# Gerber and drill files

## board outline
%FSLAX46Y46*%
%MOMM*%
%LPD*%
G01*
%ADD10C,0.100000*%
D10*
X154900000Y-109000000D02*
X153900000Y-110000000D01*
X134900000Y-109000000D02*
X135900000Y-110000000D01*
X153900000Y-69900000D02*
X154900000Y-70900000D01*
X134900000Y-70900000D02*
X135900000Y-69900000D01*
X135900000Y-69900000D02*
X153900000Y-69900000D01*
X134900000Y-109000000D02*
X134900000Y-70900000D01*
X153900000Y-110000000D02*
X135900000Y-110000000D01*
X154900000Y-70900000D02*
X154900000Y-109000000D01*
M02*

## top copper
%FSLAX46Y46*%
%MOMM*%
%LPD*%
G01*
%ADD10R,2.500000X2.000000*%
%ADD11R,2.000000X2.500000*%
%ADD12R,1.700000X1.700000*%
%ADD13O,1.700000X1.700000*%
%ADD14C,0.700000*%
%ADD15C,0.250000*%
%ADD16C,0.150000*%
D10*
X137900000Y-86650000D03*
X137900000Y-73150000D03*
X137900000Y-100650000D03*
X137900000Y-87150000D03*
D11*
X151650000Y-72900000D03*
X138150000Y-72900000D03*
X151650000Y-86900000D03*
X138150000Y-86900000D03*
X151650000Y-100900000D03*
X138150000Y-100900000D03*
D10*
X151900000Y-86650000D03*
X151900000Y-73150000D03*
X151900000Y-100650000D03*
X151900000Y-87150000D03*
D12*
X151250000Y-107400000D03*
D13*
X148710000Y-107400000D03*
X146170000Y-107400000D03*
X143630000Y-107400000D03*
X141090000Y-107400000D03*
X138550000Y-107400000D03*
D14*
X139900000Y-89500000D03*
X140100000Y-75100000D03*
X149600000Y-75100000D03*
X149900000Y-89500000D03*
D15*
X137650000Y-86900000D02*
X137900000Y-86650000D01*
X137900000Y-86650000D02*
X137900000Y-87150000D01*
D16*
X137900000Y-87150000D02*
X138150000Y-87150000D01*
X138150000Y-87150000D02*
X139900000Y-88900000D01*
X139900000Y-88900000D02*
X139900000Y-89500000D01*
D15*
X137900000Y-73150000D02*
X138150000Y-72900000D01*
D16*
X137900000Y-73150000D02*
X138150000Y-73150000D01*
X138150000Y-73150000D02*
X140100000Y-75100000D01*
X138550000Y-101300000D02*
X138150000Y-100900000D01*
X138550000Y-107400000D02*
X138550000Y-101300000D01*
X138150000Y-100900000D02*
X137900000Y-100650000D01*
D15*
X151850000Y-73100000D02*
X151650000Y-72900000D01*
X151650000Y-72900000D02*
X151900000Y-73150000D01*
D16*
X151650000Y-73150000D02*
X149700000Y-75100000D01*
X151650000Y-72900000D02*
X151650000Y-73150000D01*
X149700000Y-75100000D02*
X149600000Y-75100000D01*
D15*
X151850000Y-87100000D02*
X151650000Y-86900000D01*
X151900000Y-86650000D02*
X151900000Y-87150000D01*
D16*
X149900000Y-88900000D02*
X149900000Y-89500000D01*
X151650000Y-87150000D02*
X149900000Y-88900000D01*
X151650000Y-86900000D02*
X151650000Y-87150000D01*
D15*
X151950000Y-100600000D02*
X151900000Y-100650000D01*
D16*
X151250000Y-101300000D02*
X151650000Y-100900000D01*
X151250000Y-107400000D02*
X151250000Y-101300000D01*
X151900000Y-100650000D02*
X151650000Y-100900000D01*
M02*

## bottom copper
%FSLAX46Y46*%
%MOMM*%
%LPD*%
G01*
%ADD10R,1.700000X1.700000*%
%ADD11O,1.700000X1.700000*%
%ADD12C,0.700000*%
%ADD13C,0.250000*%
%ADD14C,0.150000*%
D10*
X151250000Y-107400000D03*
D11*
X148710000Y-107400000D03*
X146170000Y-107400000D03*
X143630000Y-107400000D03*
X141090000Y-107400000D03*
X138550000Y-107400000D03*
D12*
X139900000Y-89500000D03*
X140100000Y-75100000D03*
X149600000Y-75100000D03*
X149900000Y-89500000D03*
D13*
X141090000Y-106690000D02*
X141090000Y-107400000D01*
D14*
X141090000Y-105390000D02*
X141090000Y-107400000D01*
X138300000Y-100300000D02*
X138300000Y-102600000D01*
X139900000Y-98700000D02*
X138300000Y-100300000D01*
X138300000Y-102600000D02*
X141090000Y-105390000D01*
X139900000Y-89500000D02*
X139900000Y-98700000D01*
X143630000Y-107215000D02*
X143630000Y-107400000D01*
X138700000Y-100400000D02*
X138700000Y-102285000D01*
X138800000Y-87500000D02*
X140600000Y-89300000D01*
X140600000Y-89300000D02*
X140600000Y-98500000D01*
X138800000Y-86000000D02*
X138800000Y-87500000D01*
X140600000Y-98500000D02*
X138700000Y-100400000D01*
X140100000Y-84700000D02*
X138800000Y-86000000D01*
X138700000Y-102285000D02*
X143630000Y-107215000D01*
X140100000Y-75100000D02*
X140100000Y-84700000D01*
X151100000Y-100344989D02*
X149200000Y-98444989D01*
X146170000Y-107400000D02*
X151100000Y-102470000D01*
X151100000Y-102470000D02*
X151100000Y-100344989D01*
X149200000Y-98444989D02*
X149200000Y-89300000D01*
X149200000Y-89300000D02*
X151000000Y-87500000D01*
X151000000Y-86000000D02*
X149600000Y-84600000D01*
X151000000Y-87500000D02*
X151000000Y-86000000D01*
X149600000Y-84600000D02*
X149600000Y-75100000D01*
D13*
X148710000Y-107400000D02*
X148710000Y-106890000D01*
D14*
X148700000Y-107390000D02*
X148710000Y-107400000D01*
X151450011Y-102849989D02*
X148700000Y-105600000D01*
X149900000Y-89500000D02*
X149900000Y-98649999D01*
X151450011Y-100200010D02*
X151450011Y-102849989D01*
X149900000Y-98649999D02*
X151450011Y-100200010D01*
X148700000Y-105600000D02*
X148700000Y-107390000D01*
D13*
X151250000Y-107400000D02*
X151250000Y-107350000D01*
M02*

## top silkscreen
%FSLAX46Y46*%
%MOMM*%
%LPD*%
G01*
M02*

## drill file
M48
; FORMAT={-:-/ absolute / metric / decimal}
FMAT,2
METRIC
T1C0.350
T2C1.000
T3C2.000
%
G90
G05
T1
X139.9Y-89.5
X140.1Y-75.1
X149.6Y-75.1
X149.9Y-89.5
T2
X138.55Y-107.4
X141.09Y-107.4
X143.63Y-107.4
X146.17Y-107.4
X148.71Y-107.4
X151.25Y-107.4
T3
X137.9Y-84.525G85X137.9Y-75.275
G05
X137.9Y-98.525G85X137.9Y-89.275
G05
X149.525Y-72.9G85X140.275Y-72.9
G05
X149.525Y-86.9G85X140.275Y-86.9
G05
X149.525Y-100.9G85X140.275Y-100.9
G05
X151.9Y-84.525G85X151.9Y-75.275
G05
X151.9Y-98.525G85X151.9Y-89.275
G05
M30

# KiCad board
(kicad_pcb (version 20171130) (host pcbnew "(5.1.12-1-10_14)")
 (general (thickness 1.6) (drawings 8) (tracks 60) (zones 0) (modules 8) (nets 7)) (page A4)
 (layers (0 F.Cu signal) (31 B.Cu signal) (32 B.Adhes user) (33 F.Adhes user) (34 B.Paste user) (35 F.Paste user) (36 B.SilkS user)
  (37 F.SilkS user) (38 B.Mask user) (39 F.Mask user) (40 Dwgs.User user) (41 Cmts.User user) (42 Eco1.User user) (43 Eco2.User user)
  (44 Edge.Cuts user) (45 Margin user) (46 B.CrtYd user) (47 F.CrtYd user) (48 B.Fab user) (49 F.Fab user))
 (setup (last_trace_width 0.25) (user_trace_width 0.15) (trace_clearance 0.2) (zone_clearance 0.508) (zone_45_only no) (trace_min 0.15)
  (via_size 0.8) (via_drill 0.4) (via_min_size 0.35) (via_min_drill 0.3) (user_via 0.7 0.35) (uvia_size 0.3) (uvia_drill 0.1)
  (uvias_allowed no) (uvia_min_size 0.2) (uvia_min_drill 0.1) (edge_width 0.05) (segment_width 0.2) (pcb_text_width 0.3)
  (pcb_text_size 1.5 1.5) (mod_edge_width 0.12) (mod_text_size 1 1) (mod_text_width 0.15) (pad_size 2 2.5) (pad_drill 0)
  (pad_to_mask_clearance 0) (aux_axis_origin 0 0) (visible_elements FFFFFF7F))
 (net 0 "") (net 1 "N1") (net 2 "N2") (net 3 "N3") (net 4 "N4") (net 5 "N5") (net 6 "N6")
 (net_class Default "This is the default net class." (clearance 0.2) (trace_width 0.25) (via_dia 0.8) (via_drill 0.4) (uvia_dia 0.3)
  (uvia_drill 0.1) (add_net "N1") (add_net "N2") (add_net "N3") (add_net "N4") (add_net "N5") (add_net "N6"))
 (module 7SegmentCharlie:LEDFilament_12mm (layer F.Cu) (at 137.9 79.9 90)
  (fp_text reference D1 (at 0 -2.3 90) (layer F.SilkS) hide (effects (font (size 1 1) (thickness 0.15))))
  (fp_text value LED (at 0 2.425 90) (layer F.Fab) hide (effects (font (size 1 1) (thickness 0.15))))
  (pad "" smd rect (at 6.75 0 90) (size 2 2.5) (layers F.Paste F.Mask))
  (pad "" smd rect (at -6.75 0 90) (size 2 2.5) (layers F.Paste F.Mask))
  (pad "" np_thru_hole oval (at 0 0 90) (size 11.25 2) (drill oval 11.25 2) (layers *.Cu *.Mask))
  (pad 1 smd rect (at -6.75 0 90) (size 2 2.5) (layers F.Cu) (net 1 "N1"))
  (pad 2 smd rect (at 6.75 0 90) (size 2 2.5) (layers F.Cu) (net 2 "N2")))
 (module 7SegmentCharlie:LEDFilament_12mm (layer F.Cu) (at 137.9 93.9 90)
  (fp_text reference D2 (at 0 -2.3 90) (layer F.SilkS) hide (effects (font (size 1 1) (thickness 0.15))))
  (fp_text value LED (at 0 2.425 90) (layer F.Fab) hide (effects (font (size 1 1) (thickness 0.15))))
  (pad "" smd rect (at 6.75 0 90) (size 2 2.5) (layers F.Paste F.Mask))
  (pad "" smd rect (at -6.75 0 90) (size 2 2.5) (layers F.Paste F.Mask))
  (pad "" np_thru_hole oval (at 0 0 90) (size 11.25 2) (drill oval 11.25 2) (layers *.Cu *.Mask))
  (pad 1 smd rect (at -6.75 0 90) (size 2 2.5) (layers F.Cu) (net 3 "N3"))
  (pad 2 smd rect (at 6.75 0 90) (size 2 2.5) (layers F.Cu) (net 1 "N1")))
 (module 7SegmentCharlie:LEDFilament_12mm (layer F.Cu) (at 144.9 72.9 180)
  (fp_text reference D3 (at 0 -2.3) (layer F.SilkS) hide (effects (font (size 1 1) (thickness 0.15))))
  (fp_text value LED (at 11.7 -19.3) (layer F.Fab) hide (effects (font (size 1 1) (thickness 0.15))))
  (pad "" smd rect (at 6.75 0 180) (size 2 2.5) (layers F.Paste F.Mask))
  (pad "" smd rect (at -6.75 0 180) (size 2 2.5) (layers F.Paste F.Mask))
  (pad "" np_thru_hole oval (at 0 0 180) (size 11.25 2) (drill oval 11.25 2) (layers *.Cu *.Mask))
  (pad 1 smd rect (at -6.75 0 180) (size 2 2.5) (layers F.Cu) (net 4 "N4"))
  (pad 2 smd rect (at 6.75 0 180) (size 2 2.5) (layers F.Cu) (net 2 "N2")))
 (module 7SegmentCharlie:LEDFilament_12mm (layer F.Cu) (at 144.9 86.9 180)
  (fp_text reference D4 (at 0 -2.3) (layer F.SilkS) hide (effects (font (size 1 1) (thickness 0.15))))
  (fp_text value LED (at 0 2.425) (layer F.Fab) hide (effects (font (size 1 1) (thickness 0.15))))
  (pad "" smd rect (at 6.75 0 180) (size 2 2.5) (layers F.Paste F.Mask))
  (pad "" smd rect (at -6.75 0 180) (size 2 2.5) (layers F.Paste F.Mask))
  (pad "" np_thru_hole oval (at 0 0 180) (size 11.25 2) (drill oval 11.25 2) (layers *.Cu *.Mask))
  (pad 1 smd rect (at -6.75 0 180) (size 2 2.5) (layers F.Cu) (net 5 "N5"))
  (pad 2 smd rect (at 6.75 0 180) (size 2 2.5) (layers F.Cu) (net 1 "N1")))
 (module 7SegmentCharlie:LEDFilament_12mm (layer F.Cu) (at 144.9 100.9 180)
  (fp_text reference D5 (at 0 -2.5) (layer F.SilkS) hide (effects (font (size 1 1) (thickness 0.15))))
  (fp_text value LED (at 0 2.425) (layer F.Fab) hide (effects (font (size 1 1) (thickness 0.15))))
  (pad "" smd rect (at 6.75 0 180) (size 2 2.5) (layers F.Paste F.Mask))
  (pad "" smd rect (at -6.75 0 180) (size 2 2.5) (layers F.Paste F.Mask))
  (pad "" np_thru_hole oval (at 0 0 180) (size 11.25 2) (drill oval 11.25 2) (layers *.Cu *.Mask))
  (pad 1 smd rect (at -6.75 0 180) (size 2 2.5) (layers F.Cu) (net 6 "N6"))
  (pad 2 smd rect (at 6.75 0 180) (size 2 2.5) (layers F.Cu) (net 3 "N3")))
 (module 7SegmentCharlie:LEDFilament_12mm (layer F.Cu) (at 151.9 79.9 90)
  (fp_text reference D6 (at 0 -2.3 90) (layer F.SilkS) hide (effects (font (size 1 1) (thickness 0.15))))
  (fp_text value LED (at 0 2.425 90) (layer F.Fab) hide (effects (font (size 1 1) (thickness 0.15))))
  (pad "" smd rect (at 6.75 0 90) (size 2 2.5) (layers F.Paste F.Mask))
  (pad "" smd rect (at -6.75 0 90) (size 2 2.5) (layers F.Paste F.Mask))
  (pad "" np_thru_hole oval (at 0 0 90) (size 11.25 2) (drill oval 11.25 2) (layers *.Cu *.Mask))
  (pad 1 smd rect (at -6.75 0 90) (size 2 2.5) (layers F.Cu) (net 5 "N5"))
  (pad 2 smd rect (at 6.75 0 90) (size 2 2.5) (layers F.Cu) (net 4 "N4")))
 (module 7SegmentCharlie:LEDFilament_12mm (layer F.Cu) (at 151.9 93.9 90)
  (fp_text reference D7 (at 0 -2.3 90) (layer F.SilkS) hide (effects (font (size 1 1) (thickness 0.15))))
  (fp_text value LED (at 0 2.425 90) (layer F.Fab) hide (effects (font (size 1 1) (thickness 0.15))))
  (pad "" smd rect (at 6.75 0 90) (size 2 2.5) (layers F.Paste F.Mask))
  (pad "" smd rect (at -6.75 0 90) (size 2 2.5) (layers F.Paste F.Mask))
  (pad "" np_thru_hole oval (at 0 0 90) (size 11.25 2) (drill oval 11.25 2) (layers *.Cu *.Mask))
  (pad 1 smd rect (at -6.75 0 90) (size 2 2.5) (layers F.Cu) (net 6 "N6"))
  (pad 2 smd rect (at 6.75 0 90) (size 2 2.5) (layers F.Cu) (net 5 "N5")))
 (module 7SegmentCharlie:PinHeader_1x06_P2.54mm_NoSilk (layer F.Cu) (at 151.25 107.4 270)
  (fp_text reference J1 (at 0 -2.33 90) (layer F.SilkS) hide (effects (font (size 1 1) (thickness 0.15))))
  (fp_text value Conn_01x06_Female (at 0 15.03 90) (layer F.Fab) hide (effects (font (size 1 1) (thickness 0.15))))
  (pad 1 thru_hole rect (at 0 0 270) (size 1.7 1.7) (drill 1) (layers *.Cu *.Mask) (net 6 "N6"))
  (pad 2 thru_hole oval (at 0 2.54 270) (size 1.7 1.7) (drill 1) (layers *.Cu *.Mask) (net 5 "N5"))
  (pad 3 thru_hole oval (at 0 5.08 270) (size 1.7 1.7) (drill 1) (layers *.Cu *.Mask) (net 4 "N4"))
  (pad 4 thru_hole oval (at 0 7.62 270) (size 1.7 1.7) (drill 1) (layers *.Cu *.Mask) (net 2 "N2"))
  (pad 5 thru_hole oval (at 0 10.16 270) (size 1.7 1.7) (drill 1) (layers *.Cu *.Mask) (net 1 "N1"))
  (pad 6 thru_hole oval (at 0 12.7 270) (size 1.7 1.7) (drill 1) (layers *.Cu *.Mask) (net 3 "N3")))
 (gr_line (start 154.9 109) (end 153.9 110) (layer Edge.Cuts) (width 0.1))
 (gr_line (start 134.9 109) (end 135.9 110) (layer Edge.Cuts) (width 0.1))
 (gr_line (start 153.9 69.9) (end 154.9 70.9) (layer Edge.Cuts) (width 0.1))
 (gr_line (start 134.9 70.9) (end 135.9 69.9) (layer Edge.Cuts) (width 0.1))
 (gr_line (start 135.9 69.9) (end 153.9 69.9) (layer Edge.Cuts) (width 0.1))
 (gr_line (start 134.9 109) (end 134.9 70.9) (layer Edge.Cuts) (width 0.1))
 (gr_line (start 153.9 110) (end 135.9 110) (layer Edge.Cuts) (width 0.1))
 (gr_line (start 154.9 70.9) (end 154.9 109) (layer Edge.Cuts) (width 0.1))
 (segment (start 137.65 86.9) (end 137.9 86.65) (width 0.25) (layer F.Cu) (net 1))
 (segment (start 137.9 86.65) (end 137.9 87.15) (width 0.25) (layer F.Cu) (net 1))
 (segment (start 141.09 106.69) (end 141.09 107.4) (width 0.25) (layer B.Cu) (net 1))
 (via (at 139.9 89.5) (size 0.7) (drill 0.35) (layers F.Cu B.Cu) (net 1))
 (segment (start 137.9 87.15) (end 138.15 87.15) (width 0.15) (layer F.Cu) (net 1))
 (segment (start 138.15 87.15) (end 139.9 88.9) (width 0.15) (layer F.Cu) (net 1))
 (segment (start 139.9 88.9) (end 139.9 89.5) (width 0.15) (layer F.Cu) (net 1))
 (segment (start 141.09 105.39) (end 141.09 107.4) (width 0.15) (layer B.Cu) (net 1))
 (segment (start 138.3 100.3) (end 138.3 102.6) (width 0.15) (layer B.Cu) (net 1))
 (segment (start 139.9 98.7) (end 138.3 100.3) (width 0.15) (layer B.Cu) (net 1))
 (segment (start 138.3 102.6) (end 141.09 105.39) (width 0.15) (layer B.Cu) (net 1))
 (segment (start 139.9 89.5) (end 139.9 98.7) (width 0.15) (layer B.Cu) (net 1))
 (segment (start 137.9 73.15) (end 138.15 72.9) (width 0.25) (layer F.Cu) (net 2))
 (segment (start 137.9 73.15) (end 138.15 73.15) (width 0.15) (layer F.Cu) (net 2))
 (via (at 140.1 75.1) (size 0.7) (drill 0.35) (layers F.Cu B.Cu) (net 2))
 (segment (start 138.15 73.15) (end 140.1 75.1) (width 0.15) (layer F.Cu) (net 2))
 (segment (start 143.63 107.215) (end 143.63 107.4) (width 0.15) (layer B.Cu) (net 2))
 (segment (start 138.7 100.4) (end 138.7 102.285) (width 0.15) (layer B.Cu) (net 2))
 (segment (start 138.8 87.5) (end 140.6 89.3) (width 0.15) (layer B.Cu) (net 2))
 (segment (start 140.6 89.3) (end 140.6 98.5) (width 0.15) (layer B.Cu) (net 2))
 (segment (start 138.8 86) (end 138.8 87.5) (width 0.15) (layer B.Cu) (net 2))
 (segment (start 140.6 98.5) (end 138.7 100.4) (width 0.15) (layer B.Cu) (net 2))
 (segment (start 140.1 84.7) (end 138.8 86) (width 0.15) (layer B.Cu) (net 2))
 (segment (start 138.7 102.285) (end 143.63 107.215) (width 0.15) (layer B.Cu) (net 2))
 (segment (start 140.1 75.1) (end 140.1 84.7) (width 0.15) (layer B.Cu) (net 2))
 (segment (start 138.55 101.3) (end 138.15 100.9) (width 0.15) (layer F.Cu) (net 3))
 (segment (start 138.55 107.4) (end 138.55 101.3) (width 0.15) (layer F.Cu) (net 3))
 (segment (start 138.15 100.9) (end 137.9 100.65) (width 0.15) (layer F.Cu) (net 3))
 (segment (start 151.85 73.1) (end 151.65 72.9) (width 0.25) (layer F.Cu) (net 4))
 (segment (start 151.65 72.9) (end 151.9 73.15) (width 0.25) (layer F.Cu) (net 4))
 (via (at 149.6 75.1) (size 0.7) (drill 0.35) (layers F.Cu B.Cu) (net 4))
 (segment (start 151.65 73.15) (end 149.7 75.1) (width 0.15) (layer F.Cu) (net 4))
 (segment (start 151.65 72.9) (end 151.65 73.15) (width 0.15) (layer F.Cu) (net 4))
 (segment (start 149.7 75.1) (end 149.6 75.1) (width 0.15) (layer F.Cu) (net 4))
 (segment (start 151.1 100.344989) (end 149.2 98.444989) (width 0.15) (layer B.Cu) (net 4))
 (segment (start 146.17 107.4) (end 151.1 102.47) (width 0.15) (layer B.Cu) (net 4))
 (segment (start 151.1 102.47) (end 151.1 100.344989) (width 0.15) (layer B.Cu) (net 4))
 (segment (start 149.2 98.444989) (end 149.2 89.3) (width 0.15) (layer B.Cu) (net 4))
 (segment (start 149.2 89.3) (end 151 87.5) (width 0.15) (layer B.Cu) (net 4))
 (segment (start 151 86) (end 149.6 84.6) (width 0.15) (layer B.Cu) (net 4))
 (segment (start 151 87.5) (end 151 86) (width 0.15) (layer B.Cu) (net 4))
 (segment (start 149.6 84.6) (end 149.6 75.1) (width 0.15) (layer B.Cu) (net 4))
 (segment (start 151.85 87.1) (end 151.65 86.9) (width 0.25) (layer F.Cu) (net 5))
 (segment (start 151.9 86.65) (end 151.9 87.15) (width 0.25) (layer F.Cu) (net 5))
 (segment (start 148.71 107.4) (end 148.71 106.89) (width 0.25) (layer B.Cu) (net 5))
 (segment (start 149.9 88.9) (end 149.9 89.5) (width 0.15) (layer F.Cu) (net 5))
 (segment (start 151.65 87.15) (end 149.9 88.9) (width 0.15) (layer F.Cu) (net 5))
 (segment (start 151.65 86.9) (end 151.65 87.15) (width 0.15) (layer F.Cu) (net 5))
 (via (at 149.9 89.5) (size 0.7) (drill 0.35) (layers F.Cu B.Cu) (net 5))
 (segment (start 148.7 107.39) (end 148.71 107.4) (width 0.15) (layer B.Cu) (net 5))
 (segment (start 151.450011 102.849989) (end 148.7 105.6) (width 0.15) (layer B.Cu) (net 5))
 (segment (start 149.9 89.5) (end 149.9 98.649999) (width 0.15) (layer B.Cu) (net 5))
 (segment (start 151.450011 100.20001) (end 151.450011 102.849989) (width 0.15) (layer B.Cu) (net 5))
 (segment (start 149.9 98.649999) (end 151.450011 100.20001) (width 0.15) (layer B.Cu) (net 5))
 (segment (start 148.7 105.6) (end 148.7 107.39) (width 0.15) (layer B.Cu) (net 5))
 (segment (start 151.95 100.6) (end 151.9 100.65) (width 0.25) (layer F.Cu) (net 6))
 (segment (start 151.25 107.4) (end 151.25 107.35) (width 0.25) (layer B.Cu) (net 6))
 (segment (start 151.25 101.3) (end 151.65 100.9) (width 0.15) (layer F.Cu) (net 6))
 (segment (start 151.25 107.4) (end 151.25 101.3) (width 0.15) (layer F.Cu) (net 6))
 (segment (start 151.9 100.65) (end 151.65 100.9) (width 0.15) (layer F.Cu) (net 6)))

